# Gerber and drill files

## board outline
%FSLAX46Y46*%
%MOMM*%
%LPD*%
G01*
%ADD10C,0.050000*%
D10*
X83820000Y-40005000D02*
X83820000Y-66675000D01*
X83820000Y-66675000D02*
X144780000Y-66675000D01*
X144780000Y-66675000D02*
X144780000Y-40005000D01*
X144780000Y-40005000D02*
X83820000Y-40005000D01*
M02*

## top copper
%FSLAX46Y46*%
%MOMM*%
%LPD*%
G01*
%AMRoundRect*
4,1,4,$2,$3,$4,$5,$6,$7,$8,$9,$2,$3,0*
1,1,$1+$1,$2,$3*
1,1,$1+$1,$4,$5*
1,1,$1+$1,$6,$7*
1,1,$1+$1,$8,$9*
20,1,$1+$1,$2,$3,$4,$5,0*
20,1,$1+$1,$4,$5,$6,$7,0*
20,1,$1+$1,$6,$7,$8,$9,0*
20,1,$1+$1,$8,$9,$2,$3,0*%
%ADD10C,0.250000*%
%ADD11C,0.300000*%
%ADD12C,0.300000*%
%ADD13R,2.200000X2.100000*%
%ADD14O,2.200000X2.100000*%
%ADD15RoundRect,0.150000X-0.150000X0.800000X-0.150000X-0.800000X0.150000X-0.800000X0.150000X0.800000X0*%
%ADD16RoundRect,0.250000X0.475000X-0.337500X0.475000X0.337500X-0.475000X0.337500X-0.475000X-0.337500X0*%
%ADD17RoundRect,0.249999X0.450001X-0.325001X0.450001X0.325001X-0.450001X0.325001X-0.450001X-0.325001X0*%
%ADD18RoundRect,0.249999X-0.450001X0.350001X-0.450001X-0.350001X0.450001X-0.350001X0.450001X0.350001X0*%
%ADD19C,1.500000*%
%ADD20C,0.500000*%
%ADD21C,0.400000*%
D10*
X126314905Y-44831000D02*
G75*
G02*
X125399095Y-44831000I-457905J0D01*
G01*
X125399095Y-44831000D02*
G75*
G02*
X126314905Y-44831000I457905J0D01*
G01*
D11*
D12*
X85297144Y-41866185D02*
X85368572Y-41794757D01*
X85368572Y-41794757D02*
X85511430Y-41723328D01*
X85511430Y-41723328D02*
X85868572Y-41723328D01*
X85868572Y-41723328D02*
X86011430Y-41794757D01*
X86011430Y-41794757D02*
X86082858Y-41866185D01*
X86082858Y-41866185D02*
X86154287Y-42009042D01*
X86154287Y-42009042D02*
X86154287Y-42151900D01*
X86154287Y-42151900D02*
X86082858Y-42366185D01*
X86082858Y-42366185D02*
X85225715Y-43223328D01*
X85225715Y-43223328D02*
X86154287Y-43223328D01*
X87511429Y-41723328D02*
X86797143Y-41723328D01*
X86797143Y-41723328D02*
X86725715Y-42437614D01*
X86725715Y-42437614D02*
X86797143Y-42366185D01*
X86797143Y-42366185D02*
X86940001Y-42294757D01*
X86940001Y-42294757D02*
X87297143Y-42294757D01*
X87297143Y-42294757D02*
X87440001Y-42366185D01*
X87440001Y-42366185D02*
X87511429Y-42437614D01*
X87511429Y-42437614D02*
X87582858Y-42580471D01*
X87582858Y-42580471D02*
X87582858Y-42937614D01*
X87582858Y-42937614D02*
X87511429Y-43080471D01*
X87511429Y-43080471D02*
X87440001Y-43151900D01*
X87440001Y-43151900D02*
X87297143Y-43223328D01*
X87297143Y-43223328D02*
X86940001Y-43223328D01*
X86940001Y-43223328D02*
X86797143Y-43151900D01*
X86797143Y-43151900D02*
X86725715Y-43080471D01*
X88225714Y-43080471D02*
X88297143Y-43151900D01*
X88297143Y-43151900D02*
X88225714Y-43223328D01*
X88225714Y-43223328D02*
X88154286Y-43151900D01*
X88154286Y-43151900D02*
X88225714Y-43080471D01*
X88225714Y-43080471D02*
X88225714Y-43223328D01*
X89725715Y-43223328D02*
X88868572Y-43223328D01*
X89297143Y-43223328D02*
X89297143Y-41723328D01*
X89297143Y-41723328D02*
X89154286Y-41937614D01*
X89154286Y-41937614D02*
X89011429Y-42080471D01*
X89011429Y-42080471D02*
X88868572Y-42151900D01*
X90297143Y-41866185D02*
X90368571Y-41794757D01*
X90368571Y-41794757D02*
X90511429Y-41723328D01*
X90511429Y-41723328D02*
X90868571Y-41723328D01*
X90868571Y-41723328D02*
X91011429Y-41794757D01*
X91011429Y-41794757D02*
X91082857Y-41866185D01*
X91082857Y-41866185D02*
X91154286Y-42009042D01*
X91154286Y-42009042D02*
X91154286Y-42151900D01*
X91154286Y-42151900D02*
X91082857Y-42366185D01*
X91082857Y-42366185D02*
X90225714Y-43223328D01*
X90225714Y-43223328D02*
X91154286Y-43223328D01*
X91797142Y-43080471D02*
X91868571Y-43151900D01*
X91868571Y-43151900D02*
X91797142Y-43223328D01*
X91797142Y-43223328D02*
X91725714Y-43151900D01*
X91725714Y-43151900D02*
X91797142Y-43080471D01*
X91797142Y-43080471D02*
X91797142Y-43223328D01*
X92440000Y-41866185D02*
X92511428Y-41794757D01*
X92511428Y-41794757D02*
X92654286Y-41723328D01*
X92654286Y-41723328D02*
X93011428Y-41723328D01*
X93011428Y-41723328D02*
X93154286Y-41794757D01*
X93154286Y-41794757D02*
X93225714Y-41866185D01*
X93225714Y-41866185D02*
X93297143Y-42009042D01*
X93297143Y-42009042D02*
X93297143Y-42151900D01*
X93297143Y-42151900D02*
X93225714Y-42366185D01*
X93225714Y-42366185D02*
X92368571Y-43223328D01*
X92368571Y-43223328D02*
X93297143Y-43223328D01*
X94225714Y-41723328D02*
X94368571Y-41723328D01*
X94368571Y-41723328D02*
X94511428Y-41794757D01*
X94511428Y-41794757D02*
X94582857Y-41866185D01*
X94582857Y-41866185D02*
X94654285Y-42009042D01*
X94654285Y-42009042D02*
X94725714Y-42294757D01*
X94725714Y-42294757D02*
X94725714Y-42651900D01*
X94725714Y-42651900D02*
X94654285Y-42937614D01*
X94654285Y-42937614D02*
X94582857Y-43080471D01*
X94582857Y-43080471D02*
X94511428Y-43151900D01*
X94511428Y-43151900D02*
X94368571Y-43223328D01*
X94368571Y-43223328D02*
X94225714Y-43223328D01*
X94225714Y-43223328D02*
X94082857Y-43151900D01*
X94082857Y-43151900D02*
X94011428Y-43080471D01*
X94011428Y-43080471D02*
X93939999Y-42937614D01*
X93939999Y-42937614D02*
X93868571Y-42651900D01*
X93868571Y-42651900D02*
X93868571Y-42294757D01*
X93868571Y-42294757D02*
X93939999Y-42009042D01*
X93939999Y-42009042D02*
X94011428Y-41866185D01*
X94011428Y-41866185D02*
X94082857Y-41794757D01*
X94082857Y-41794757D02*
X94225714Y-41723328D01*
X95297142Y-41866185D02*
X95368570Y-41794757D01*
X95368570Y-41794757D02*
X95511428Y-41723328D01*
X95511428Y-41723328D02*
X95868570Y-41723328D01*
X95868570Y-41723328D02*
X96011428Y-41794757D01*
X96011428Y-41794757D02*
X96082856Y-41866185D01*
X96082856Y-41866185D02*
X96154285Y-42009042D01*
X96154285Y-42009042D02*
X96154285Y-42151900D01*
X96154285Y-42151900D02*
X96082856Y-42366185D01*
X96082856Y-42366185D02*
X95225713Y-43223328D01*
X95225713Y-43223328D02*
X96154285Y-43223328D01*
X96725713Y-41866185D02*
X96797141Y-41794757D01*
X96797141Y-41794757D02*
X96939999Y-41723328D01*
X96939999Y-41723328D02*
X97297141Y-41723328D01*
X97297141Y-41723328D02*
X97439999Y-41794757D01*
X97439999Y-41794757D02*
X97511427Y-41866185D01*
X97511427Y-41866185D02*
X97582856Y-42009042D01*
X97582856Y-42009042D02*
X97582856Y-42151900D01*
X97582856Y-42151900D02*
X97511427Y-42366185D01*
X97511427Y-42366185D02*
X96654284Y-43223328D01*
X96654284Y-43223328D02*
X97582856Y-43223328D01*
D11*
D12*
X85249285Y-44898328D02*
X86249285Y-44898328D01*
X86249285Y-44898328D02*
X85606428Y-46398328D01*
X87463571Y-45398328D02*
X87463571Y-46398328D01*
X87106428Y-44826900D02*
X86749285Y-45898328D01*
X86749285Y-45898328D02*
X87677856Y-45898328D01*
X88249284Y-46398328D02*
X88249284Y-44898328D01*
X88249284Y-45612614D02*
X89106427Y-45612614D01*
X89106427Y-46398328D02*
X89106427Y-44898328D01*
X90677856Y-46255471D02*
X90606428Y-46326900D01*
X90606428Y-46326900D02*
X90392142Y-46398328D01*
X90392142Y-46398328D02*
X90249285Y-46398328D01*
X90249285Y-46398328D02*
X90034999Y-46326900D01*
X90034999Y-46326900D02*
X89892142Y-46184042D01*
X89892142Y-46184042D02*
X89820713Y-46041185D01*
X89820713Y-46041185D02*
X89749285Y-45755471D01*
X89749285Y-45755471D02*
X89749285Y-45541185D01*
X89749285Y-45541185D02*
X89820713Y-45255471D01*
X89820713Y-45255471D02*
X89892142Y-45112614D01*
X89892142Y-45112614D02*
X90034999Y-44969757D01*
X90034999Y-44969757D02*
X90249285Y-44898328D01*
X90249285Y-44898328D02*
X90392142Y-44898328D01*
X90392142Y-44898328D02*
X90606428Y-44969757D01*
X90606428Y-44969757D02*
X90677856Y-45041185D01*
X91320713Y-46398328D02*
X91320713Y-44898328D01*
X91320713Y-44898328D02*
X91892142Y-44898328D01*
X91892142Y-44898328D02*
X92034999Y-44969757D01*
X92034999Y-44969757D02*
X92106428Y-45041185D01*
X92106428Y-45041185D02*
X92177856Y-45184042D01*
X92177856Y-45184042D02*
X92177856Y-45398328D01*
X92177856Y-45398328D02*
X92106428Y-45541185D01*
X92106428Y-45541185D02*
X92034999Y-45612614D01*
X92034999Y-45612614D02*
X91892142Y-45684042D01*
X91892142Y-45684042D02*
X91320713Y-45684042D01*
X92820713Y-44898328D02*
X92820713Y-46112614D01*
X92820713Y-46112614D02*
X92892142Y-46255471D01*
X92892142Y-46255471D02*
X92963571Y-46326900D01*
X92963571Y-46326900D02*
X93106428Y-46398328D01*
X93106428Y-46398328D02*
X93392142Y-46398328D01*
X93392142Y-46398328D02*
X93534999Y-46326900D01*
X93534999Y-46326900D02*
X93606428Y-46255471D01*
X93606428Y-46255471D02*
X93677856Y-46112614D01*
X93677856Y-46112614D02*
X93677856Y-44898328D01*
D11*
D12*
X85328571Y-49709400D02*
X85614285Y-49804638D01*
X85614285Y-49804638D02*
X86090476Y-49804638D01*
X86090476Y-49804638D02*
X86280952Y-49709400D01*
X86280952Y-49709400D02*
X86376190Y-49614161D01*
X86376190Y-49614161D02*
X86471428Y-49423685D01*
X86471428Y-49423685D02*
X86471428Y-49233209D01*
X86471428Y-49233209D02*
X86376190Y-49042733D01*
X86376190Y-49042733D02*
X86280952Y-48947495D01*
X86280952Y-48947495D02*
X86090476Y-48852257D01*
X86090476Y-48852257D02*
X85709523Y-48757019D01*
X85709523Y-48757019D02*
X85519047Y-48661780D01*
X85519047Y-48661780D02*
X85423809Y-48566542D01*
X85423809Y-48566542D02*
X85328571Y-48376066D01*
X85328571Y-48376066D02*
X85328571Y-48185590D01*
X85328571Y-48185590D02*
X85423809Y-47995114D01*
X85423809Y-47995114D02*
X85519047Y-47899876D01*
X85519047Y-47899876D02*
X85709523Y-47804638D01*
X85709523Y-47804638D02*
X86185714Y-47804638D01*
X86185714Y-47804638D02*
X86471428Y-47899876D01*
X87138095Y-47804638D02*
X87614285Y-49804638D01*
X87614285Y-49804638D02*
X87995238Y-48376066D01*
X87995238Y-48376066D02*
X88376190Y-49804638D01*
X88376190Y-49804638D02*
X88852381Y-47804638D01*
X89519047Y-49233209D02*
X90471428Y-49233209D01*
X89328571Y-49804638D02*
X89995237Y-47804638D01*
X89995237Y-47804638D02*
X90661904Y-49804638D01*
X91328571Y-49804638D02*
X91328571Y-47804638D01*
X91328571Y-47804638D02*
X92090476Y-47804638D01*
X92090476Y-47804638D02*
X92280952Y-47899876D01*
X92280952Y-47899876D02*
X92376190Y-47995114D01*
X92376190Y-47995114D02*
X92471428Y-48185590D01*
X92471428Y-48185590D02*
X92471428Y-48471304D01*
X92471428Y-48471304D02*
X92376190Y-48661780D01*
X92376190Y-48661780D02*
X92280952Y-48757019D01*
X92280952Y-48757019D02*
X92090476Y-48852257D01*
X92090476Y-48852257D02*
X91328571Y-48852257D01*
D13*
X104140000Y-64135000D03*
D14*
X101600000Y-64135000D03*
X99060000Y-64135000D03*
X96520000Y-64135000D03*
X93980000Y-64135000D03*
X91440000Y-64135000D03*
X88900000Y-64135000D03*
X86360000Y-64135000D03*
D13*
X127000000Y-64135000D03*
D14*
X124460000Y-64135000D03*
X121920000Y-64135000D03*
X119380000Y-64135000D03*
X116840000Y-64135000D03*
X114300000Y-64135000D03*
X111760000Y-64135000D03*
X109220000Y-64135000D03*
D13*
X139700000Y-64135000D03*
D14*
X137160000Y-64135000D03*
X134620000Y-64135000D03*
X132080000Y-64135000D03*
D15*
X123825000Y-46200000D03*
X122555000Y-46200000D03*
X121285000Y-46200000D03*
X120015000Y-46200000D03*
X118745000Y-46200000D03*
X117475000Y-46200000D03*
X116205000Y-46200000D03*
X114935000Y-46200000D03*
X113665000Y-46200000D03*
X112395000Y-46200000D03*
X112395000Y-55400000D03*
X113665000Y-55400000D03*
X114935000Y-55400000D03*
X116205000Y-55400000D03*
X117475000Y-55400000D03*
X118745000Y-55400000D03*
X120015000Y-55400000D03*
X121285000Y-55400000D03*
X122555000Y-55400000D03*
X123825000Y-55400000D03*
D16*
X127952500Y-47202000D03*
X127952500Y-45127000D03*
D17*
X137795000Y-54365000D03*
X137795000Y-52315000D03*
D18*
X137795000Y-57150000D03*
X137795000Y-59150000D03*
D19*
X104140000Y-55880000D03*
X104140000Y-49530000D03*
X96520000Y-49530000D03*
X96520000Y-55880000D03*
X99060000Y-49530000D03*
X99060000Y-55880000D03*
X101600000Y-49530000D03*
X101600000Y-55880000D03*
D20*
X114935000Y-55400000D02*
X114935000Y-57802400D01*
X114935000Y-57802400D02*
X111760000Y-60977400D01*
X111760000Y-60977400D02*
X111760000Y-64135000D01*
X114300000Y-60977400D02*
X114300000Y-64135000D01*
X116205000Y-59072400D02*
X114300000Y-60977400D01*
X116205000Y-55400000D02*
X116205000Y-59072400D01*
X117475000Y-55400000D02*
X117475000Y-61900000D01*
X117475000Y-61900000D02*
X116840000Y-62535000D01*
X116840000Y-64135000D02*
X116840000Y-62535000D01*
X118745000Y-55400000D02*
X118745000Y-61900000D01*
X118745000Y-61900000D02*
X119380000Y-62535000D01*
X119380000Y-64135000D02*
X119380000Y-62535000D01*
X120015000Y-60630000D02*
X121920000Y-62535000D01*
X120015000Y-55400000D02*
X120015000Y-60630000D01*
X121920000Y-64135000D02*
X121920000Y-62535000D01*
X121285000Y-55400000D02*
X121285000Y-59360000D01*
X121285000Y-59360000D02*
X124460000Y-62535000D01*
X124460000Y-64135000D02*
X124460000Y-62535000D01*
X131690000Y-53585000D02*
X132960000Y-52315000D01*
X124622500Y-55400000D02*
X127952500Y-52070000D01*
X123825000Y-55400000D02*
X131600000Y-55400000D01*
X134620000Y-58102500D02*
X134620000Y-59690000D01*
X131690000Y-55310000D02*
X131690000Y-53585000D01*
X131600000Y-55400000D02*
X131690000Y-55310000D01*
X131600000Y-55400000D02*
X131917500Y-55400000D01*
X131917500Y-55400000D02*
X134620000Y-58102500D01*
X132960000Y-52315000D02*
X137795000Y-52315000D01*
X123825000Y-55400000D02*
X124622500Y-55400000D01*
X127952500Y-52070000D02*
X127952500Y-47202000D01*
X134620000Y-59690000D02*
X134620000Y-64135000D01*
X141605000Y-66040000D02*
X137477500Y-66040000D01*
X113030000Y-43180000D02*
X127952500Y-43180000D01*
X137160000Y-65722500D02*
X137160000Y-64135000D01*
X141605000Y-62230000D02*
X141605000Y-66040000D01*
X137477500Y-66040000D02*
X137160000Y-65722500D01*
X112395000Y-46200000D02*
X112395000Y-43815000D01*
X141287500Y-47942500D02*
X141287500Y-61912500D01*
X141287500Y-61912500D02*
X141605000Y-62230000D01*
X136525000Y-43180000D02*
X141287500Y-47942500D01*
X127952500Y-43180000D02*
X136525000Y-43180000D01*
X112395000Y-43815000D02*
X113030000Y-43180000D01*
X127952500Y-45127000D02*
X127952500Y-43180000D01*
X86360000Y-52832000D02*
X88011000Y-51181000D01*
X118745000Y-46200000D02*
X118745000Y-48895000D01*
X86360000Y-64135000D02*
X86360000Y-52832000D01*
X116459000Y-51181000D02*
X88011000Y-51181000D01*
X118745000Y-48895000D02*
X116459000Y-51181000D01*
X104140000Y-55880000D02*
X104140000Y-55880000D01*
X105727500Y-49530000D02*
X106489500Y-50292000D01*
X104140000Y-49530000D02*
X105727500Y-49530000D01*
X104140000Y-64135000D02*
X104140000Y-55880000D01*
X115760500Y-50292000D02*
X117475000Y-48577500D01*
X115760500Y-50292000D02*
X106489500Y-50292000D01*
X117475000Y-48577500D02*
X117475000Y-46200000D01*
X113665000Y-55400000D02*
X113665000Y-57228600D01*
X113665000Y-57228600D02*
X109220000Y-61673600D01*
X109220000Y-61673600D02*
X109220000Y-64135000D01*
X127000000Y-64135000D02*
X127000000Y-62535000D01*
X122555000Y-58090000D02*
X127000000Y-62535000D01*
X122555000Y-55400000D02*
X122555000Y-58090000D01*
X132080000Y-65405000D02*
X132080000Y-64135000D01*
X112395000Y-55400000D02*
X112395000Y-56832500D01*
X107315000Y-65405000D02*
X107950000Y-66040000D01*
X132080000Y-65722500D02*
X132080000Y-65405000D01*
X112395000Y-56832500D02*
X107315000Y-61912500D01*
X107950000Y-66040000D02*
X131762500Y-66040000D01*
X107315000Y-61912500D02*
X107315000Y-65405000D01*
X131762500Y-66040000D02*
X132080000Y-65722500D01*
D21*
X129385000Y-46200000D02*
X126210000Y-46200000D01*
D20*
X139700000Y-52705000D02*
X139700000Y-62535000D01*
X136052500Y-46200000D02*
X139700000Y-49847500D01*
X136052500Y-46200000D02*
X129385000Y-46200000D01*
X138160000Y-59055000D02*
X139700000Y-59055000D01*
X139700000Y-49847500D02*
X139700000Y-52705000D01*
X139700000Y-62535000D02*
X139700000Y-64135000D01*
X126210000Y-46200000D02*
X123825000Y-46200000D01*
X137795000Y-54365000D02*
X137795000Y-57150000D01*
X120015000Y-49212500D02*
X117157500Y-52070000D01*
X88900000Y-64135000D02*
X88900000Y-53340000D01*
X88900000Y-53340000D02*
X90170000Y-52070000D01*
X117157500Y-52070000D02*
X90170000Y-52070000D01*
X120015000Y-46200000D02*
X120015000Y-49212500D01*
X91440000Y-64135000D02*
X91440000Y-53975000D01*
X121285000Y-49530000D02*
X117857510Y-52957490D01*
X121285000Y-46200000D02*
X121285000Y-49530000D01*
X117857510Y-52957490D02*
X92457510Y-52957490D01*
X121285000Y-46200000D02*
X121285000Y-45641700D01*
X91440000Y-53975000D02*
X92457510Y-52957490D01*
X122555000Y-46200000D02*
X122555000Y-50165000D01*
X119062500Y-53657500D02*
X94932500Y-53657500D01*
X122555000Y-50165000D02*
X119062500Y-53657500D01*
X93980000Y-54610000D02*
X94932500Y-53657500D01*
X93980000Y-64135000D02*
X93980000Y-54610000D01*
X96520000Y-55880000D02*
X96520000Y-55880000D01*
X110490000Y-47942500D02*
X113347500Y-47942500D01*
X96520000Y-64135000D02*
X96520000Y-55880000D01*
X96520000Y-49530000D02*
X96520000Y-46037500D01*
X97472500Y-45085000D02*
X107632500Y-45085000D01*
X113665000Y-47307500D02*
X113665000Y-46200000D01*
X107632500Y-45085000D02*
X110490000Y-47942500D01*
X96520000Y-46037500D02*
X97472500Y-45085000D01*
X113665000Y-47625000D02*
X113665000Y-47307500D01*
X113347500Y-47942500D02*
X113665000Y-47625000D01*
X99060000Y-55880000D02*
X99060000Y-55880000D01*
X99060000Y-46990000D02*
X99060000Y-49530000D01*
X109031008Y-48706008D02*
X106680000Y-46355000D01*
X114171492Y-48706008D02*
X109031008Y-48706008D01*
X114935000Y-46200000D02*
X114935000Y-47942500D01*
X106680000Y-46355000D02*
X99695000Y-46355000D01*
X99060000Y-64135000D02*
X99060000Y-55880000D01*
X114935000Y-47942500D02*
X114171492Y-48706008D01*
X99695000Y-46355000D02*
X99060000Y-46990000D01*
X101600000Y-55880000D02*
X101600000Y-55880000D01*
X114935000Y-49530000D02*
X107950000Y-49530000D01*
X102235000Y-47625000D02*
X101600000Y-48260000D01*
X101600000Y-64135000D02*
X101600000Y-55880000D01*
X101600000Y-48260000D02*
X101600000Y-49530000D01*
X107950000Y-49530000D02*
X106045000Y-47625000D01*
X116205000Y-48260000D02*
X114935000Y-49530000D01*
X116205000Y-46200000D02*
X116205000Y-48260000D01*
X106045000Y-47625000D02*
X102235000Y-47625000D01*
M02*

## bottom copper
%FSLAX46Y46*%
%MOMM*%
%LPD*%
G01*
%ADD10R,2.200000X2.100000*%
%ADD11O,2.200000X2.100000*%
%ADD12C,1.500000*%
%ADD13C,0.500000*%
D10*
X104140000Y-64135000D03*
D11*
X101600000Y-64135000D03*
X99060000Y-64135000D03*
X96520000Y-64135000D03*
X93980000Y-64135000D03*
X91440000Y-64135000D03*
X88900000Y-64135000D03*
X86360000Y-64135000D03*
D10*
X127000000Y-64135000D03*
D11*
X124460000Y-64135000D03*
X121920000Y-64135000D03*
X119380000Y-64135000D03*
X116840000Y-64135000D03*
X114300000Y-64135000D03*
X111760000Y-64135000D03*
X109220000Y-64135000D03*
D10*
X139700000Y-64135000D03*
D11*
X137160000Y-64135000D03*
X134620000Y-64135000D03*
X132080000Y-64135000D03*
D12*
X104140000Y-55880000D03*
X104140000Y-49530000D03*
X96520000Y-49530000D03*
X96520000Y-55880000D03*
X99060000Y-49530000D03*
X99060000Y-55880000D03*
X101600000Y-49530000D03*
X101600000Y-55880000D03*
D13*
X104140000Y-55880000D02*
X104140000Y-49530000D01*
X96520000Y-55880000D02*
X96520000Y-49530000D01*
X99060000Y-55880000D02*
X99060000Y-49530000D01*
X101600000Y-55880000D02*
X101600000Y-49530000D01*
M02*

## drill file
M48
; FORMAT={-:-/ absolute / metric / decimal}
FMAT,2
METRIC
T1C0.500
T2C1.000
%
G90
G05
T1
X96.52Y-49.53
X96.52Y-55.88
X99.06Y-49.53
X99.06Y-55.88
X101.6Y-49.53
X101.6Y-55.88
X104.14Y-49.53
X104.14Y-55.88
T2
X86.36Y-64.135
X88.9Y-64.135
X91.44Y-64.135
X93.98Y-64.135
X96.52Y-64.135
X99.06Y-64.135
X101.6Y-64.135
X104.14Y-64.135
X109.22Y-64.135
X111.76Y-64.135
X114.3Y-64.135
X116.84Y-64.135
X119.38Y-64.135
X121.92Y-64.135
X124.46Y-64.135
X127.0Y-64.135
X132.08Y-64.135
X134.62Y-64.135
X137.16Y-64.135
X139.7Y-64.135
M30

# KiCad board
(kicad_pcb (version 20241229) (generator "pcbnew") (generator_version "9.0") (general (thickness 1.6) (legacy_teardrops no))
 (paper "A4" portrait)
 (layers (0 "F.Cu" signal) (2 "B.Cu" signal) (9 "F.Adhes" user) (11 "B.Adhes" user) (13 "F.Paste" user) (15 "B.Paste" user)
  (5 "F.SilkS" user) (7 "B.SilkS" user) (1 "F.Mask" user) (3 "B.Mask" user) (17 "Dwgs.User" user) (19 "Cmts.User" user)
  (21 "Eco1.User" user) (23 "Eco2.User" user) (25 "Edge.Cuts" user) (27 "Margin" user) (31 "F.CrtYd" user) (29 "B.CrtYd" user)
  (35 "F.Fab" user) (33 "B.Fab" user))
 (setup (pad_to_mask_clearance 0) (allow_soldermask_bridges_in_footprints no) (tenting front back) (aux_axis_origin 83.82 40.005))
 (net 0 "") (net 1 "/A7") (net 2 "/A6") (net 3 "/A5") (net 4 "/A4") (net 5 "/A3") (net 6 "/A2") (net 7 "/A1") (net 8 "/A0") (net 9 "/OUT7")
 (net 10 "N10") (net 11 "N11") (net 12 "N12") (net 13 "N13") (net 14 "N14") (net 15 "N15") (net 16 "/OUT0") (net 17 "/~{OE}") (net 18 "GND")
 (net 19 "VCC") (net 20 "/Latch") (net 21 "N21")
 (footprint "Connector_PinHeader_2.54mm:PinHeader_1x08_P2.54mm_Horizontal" (layer "F.Cu") (at 104.14 64.135 -90)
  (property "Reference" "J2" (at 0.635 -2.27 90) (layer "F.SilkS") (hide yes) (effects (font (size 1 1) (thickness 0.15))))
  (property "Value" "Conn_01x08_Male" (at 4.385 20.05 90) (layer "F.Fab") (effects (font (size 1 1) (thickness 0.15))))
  (pad "1" thru_hole rect (at 0 0 270) (size 2.1 2.2) (drill 1) (layers "*.Cu" "*.Mask") (remove_unused_layers no) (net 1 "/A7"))
  (pad "2" thru_hole oval (at 0 2.54 270) (size 2.1 2.2) (drill 1) (layers "*.Cu" "*.Mask") (remove_unused_layers no) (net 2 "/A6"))
  (pad "3" thru_hole oval (at 0 5.08 270) (size 2.1 2.2) (drill 1) (layers "*.Cu" "*.Mask") (remove_unused_layers no) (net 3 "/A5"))
  (pad "4" thru_hole oval (at 0 7.62 270) (size 2.1 2.2) (drill 1) (layers "*.Cu" "*.Mask") (remove_unused_layers no) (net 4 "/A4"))
  (pad "5" thru_hole oval (at 0 10.16 270) (size 2.1 2.2) (drill 1) (layers "*.Cu" "*.Mask") (remove_unused_layers no) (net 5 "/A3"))
  (pad "6" thru_hole oval (at 0 12.7 270) (size 2.1 2.2) (drill 1) (layers "*.Cu" "*.Mask") (remove_unused_layers no) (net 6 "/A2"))
  (pad "7" thru_hole oval (at 0 15.24 270) (size 2.1 2.2) (drill 1) (layers "*.Cu" "*.Mask") (remove_unused_layers no) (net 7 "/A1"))
  (pad "8" thru_hole oval (at 0 17.78 270) (size 2.1 2.2) (drill 1) (layers "*.Cu" "*.Mask") (remove_unused_layers no) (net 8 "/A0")))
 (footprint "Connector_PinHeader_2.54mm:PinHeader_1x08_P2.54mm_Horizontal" (layer "F.Cu") (at 127 64.135 -90)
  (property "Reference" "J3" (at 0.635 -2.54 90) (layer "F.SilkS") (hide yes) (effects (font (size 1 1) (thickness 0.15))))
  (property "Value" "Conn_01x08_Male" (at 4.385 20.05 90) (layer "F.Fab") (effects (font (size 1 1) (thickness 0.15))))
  (pad "1" thru_hole rect (at 0 0 270) (size 2.1 2.2) (drill 1) (layers "*.Cu" "*.Mask") (remove_unused_layers no) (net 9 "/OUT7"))
  (pad "2" thru_hole oval (at 0 2.54 270) (size 2.1 2.2) (drill 1) (layers "*.Cu" "*.Mask") (remove_unused_layers no) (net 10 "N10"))
  (pad "3" thru_hole oval (at 0 5.08 270) (size 2.1 2.2) (drill 1) (layers "*.Cu" "*.Mask") (remove_unused_layers no) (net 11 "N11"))
  (pad "4" thru_hole oval (at 0 7.62 270) (size 2.1 2.2) (drill 1) (layers "*.Cu" "*.Mask") (remove_unused_layers no) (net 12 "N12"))
  (pad "5" thru_hole oval (at 0 10.16 270) (size 2.1 2.2) (drill 1) (layers "*.Cu" "*.Mask") (remove_unused_layers no) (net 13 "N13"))
  (pad "6" thru_hole oval (at 0 12.7 270) (size 2.1 2.2) (drill 1) (layers "*.Cu" "*.Mask") (remove_unused_layers no) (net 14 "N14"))
  (pad "7" thru_hole oval (at 0 15.24 270) (size 2.1 2.2) (drill 1) (layers "*.Cu" "*.Mask") (remove_unused_layers no) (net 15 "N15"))
  (pad "8" thru_hole oval (at 0 17.78 270) (size 2.1 2.2) (drill 1) (layers "*.Cu" "*.Mask") (remove_unused_layers no) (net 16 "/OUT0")))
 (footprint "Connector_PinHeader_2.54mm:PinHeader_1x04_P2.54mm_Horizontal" (layer "F.Cu") (at 139.7 64.135 -90)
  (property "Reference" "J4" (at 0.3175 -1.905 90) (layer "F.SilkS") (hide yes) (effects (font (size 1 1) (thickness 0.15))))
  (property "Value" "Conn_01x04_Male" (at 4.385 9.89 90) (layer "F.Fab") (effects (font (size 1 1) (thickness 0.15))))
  (pad "1" thru_hole rect (at 0 0 270) (size 2.1 2.2) (drill 1) (layers "*.Cu" "*.Mask") (remove_unused_layers no) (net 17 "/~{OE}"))
  (pad "2" thru_hole oval (at 0 2.54 270) (size 2.1 2.2) (drill 1) (layers "*.Cu" "*.Mask") (remove_unused_layers no) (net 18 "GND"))
  (pad "3" thru_hole oval (at 0 5.08 270) (size 2.1 2.2) (drill 1) (layers "*.Cu" "*.Mask") (remove_unused_layers no) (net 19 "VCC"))
  (pad "4" thru_hole oval (at 0 7.62 270) (size 2.1 2.2) (drill 1) (layers "*.Cu" "*.Mask") (remove_unused_layers no) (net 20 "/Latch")))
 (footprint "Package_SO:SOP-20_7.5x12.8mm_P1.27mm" (layer "F.Cu") (at 118.11 50.8 -90)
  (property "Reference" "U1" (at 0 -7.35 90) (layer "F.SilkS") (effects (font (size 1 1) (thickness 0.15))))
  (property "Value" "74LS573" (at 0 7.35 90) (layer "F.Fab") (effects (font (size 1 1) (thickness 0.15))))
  (pad "1" smd roundrect (at -4.6 -5.715 270) (size 1.9 0.6) (layers "F.Cu" "F.Mask" "F.Paste") (roundrect_rratio 0.25) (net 17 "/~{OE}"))
  (pad "2" smd roundrect (at -4.6 -4.445 270) (size 1.9 0.6) (layers "F.Cu" "F.Mask" "F.Paste") (roundrect_rratio 0.25) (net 5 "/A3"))
  (pad "3" smd roundrect (at -4.6 -3.175 270) (size 1.9 0.6) (layers "F.Cu" "F.Mask" "F.Paste") (roundrect_rratio 0.25) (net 6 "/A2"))
  (pad "4" smd roundrect (at -4.6 -1.905 270) (size 1.9 0.6) (layers "F.Cu" "F.Mask" "F.Paste") (roundrect_rratio 0.25) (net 7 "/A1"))
  (pad "5" smd roundrect (at -4.6 -0.635 270) (size 1.9 0.6) (layers "F.Cu" "F.Mask" "F.Paste") (roundrect_rratio 0.25) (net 8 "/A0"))
  (pad "6" smd roundrect (at -4.6 0.635 270) (size 1.9 0.6) (layers "F.Cu" "F.Mask" "F.Paste") (roundrect_rratio 0.25) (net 1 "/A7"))
  (pad "7" smd roundrect (at -4.6 1.905 270) (size 1.9 0.6) (layers "F.Cu" "F.Mask" "F.Paste") (roundrect_rratio 0.25) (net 2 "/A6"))
  (pad "8" smd roundrect (at -4.6 3.175 270) (size 1.9 0.6) (layers "F.Cu" "F.Mask" "F.Paste") (roundrect_rratio 0.25) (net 3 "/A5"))
  (pad "9" smd roundrect (at -4.6 4.445 270) (size 1.9 0.6) (layers "F.Cu" "F.Mask" "F.Paste") (roundrect_rratio 0.25) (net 4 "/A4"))
  (pad "10" smd roundrect (at -4.6 5.715 270) (size 1.9 0.6) (layers "F.Cu" "F.Mask" "F.Paste") (roundrect_rratio 0.25) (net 18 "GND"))
  (pad "11" smd roundrect (at 4.6 5.715 270) (size 1.9 0.6) (layers "F.Cu" "F.Mask" "F.Paste") (roundrect_rratio 0.25) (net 20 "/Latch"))
  (pad "12" smd roundrect (at 4.6 4.445 270) (size 1.9 0.6) (layers "F.Cu" "F.Mask" "F.Paste") (roundrect_rratio 0.25) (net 16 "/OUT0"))
  (pad "13" smd roundrect (at 4.6 3.175 270) (size 1.9 0.6) (layers "F.Cu" "F.Mask" "F.Paste") (roundrect_rratio 0.25) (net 15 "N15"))
  (pad "14" smd roundrect (at 4.6 1.905 270) (size 1.9 0.6) (layers "F.Cu" "F.Mask" "F.Paste") (roundrect_rratio 0.25) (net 14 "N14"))
  (pad "15" smd roundrect (at 4.6 0.635 270) (size 1.9 0.6) (layers "F.Cu" "F.Mask" "F.Paste") (roundrect_rratio 0.25) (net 13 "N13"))
  (pad "16" smd roundrect (at 4.6 -0.635 270) (size 1.9 0.6) (layers "F.Cu" "F.Mask" "F.Paste") (roundrect_rratio 0.25) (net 12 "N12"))
  (pad "17" smd roundrect (at 4.6 -1.905 270) (size 1.9 0.6) (layers "F.Cu" "F.Mask" "F.Paste") (roundrect_rratio 0.25) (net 11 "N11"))
  (pad "18" smd roundrect (at 4.6 -3.175 270) (size 1.9 0.6) (layers "F.Cu" "F.Mask" "F.Paste") (roundrect_rratio 0.25) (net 10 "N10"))
  (pad "19" smd roundrect (at 4.6 -4.445 270) (size 1.9 0.6) (layers "F.Cu" "F.Mask" "F.Paste") (roundrect_rratio 0.25) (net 9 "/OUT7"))
  (pad "20" smd roundrect (at 4.6 -5.715 270) (size 1.9 0.6) (layers "F.Cu" "F.Mask" "F.Paste") (roundrect_rratio 0.25) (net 19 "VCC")))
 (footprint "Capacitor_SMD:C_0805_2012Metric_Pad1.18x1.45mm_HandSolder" (layer "F.Cu") (at 127.9525 46.1645 90)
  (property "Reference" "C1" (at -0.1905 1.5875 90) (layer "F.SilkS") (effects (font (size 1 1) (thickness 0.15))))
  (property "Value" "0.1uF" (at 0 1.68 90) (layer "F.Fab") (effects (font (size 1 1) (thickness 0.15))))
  (pad "1" smd roundrect (at -1.0375 0 90) (size 1.175 1.45) (layers "F.Cu" "F.Mask" "F.Paste") (roundrect_rratio 0.2127659574)
   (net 19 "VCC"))
  (pad "2" smd roundrect (at 1.0375 0 90) (size 1.175 1.45) (layers "F.Cu" "F.Mask" "F.Paste") (roundrect_rratio 0.2127659574)
   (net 18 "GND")))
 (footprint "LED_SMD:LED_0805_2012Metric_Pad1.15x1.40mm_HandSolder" (layer "F.Cu") (at 137.795 53.34 90)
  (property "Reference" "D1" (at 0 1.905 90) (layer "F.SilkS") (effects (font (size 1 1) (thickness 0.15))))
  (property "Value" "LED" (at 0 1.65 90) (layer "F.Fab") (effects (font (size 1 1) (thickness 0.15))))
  (pad "1" smd roundrect (at -1.025 0 90) (size 1.15 1.4) (layers "F.Cu" "F.Mask" "F.Paste") (roundrect_rratio 0.2173904348) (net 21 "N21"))
  (pad "2" smd roundrect (at 1.025 0 90) (size 1.15 1.4) (layers "F.Cu" "F.Mask" "F.Paste") (roundrect_rratio 0.2173904348) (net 19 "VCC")))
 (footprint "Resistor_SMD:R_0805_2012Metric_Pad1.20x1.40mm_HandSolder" (layer "F.Cu") (at 137.795 58.15 -90)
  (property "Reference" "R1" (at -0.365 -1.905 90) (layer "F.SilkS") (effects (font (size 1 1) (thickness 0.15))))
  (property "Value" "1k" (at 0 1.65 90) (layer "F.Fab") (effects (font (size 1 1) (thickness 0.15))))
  (pad "1" smd roundrect (at -1 0 270) (size 1.2 1.4) (layers "F.Cu" "F.Mask" "F.Paste") (roundrect_rratio 0.2083325) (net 21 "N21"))
  (pad "2" smd roundrect (at 1 0 270) (size 1.2 1.4) (layers "F.Cu" "F.Mask" "F.Paste") (roundrect_rratio 0.2083325) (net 17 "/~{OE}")))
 (gr_circle (center 125.857 44.831) (end 126.314905 44.831) (stroke (width 0.25) (type solid)) (fill no) (layer "F.Cu"))
 (gr_line (start 83.82 40.005) (end 83.82 66.675) (stroke (width 0.05) (type solid)) (layer "Edge.Cuts"))
 (gr_line (start 83.82 66.675) (end 144.78 66.675) (stroke (width 0.05) (type solid)) (layer "Edge.Cuts"))
 (gr_line (start 144.78 66.675) (end 144.78 40.005) (stroke (width 0.05) (type solid)) (layer "Edge.Cuts"))
 (gr_line (start 144.78 40.005) (end 83.82 40.005) (stroke (width 0.05) (type solid)) (layer "Edge.Cuts"))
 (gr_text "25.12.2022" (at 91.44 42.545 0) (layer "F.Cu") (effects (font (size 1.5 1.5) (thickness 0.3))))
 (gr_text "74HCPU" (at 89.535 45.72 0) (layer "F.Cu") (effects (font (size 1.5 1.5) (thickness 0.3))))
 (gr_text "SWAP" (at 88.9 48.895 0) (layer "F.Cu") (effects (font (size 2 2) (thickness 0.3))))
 (segment (start 114.935 55.4) (end 114.935 57.8024) (width 0.5) (layer "F.Cu") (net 15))
 (segment (start 114.935 57.8024) (end 111.76 60.9774) (width 0.5) (layer "F.Cu") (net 15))
 (segment (start 111.76 60.9774) (end 111.76 64.135) (width 0.5) (layer "F.Cu") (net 15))
 (segment (start 114.3 60.9774) (end 114.3 64.135) (width 0.5) (layer "F.Cu") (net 14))
 (segment (start 116.205 59.0724) (end 114.3 60.9774) (width 0.5) (layer "F.Cu") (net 14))
 (segment (start 116.205 55.4) (end 116.205 59.0724) (width 0.5) (layer "F.Cu") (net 14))
 (segment (start 117.475 55.4) (end 117.475 61.9) (width 0.5) (layer "F.Cu") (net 13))
 (segment (start 117.475 61.9) (end 116.84 62.535) (width 0.5) (layer "F.Cu") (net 13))
 (segment (start 116.84 64.135) (end 116.84 62.535) (width 0.5) (layer "F.Cu") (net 13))
 (segment (start 118.745 55.4) (end 118.745 61.9) (width 0.5) (layer "F.Cu") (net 12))
 (segment (start 118.745 61.9) (end 119.38 62.535) (width 0.5) (layer "F.Cu") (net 12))
 (segment (start 119.38 64.135) (end 119.38 62.535) (width 0.5) (layer "F.Cu") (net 12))
 (segment (start 120.015 60.63) (end 121.92 62.535) (width 0.5) (layer "F.Cu") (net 11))
 (segment (start 120.015 55.4) (end 120.015 60.63) (width 0.5) (layer "F.Cu") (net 11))
 (segment (start 121.92 64.135) (end 121.92 62.535) (width 0.5) (layer "F.Cu") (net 11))
 (segment (start 121.285 55.4) (end 121.285 59.36) (width 0.5) (layer "F.Cu") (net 10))
 (segment (start 121.285 59.36) (end 124.46 62.535) (width 0.5) (layer "F.Cu") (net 10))
 (segment (start 124.46 64.135) (end 124.46 62.535) (width 0.5) (layer "F.Cu") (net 10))
 (segment (start 131.69 53.585) (end 132.96 52.315) (width 0.5) (layer "F.Cu") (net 19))
 (segment (start 124.6225 55.4) (end 127.9525 52.07) (width 0.5) (layer "F.Cu") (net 19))
 (segment (start 123.825 55.4) (end 131.6 55.4) (width 0.5) (layer "F.Cu") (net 19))
 (segment (start 134.62 58.1025) (end 134.62 59.69) (width 0.5) (layer "F.Cu") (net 19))
 (segment (start 131.69 55.31) (end 131.69 53.585) (width 0.5) (layer "F.Cu") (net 19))
 (segment (start 131.6 55.4) (end 131.69 55.31) (width 0.5) (layer "F.Cu") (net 19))
 (segment (start 131.6 55.4) (end 131.9175 55.4) (width 0.5) (layer "F.Cu") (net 19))
 (segment (start 131.9175 55.4) (end 134.62 58.1025) (width 0.5) (layer "F.Cu") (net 19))
 (segment (start 132.96 52.315) (end 137.795 52.315) (width 0.5) (layer "F.Cu") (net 19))
 (segment (start 123.825 55.4) (end 124.6225 55.4) (width 0.5) (layer "F.Cu") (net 19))
 (segment (start 127.9525 52.07) (end 127.9525 47.202) (width 0.5) (layer "F.Cu") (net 19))
 (segment (start 134.62 59.69) (end 134.62 64.135) (width 0.5) (layer "F.Cu") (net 19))
 (segment (start 141.605 66.04) (end 137.4775 66.04) (width 0.5) (layer "F.Cu") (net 18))
 (segment (start 113.03 43.18) (end 127.9525 43.18) (width 0.5) (layer "F.Cu") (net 18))
 (segment (start 137.16 65.7225) (end 137.16 64.135) (width 0.5) (layer "F.Cu") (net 18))
 (segment (start 141.605 62.23) (end 141.605 66.04) (width 0.5) (layer "F.Cu") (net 18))
 (segment (start 137.4775 66.04) (end 137.16 65.7225) (width 0.5) (layer "F.Cu") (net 18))
 (segment (start 112.395 46.2) (end 112.395 43.815) (width 0.5) (layer "F.Cu") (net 18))
 (segment (start 141.2875 47.9425) (end 141.2875 61.9125) (width 0.5) (layer "F.Cu") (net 18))
 (segment (start 141.2875 61.9125) (end 141.605 62.23) (width 0.5) (layer "F.Cu") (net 18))
 (segment (start 136.525 43.18) (end 141.2875 47.9425) (width 0.5) (layer "F.Cu") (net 18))
 (segment (start 127.9525 43.18) (end 136.525 43.18) (width 0.5) (layer "F.Cu") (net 18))
 (segment (start 112.395 43.815) (end 113.03 43.18) (width 0.5) (layer "F.Cu") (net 18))
 (segment (start 127.9525 45.127) (end 127.9525 43.18) (width 0.5) (layer "F.Cu") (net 18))
 (segment (start 86.36 52.832) (end 88.011 51.181) (width 0.5) (layer "F.Cu") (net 8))
 (segment (start 118.745 46.2) (end 118.745 48.895) (width 0.5) (layer "F.Cu") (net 8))
 (segment (start 86.36 64.135) (end 86.36 52.832) (width 0.5) (layer "F.Cu") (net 8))
 (segment (start 116.459 51.181) (end 88.011 51.181) (width 0.5) (layer "F.Cu") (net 8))
 (segment (start 118.745 48.895) (end 116.459 51.181) (width 0.5) (layer "F.Cu") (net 8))
 (segment (start 104.14 55.88) (end 104.14 55.88) (width 0.5) (layer "F.Cu") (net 1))
 (segment (start 105.7275 49.53) (end 106.4895 50.292) (width 0.5) (layer "F.Cu") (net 1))
 (segment (start 104.14 49.53) (end 105.7275 49.53) (width 0.5) (layer "F.Cu") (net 1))
 (segment (start 104.14 64.135) (end 104.14 55.88) (width 0.5) (layer "F.Cu") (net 1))
 (segment (start 115.7605 50.292) (end 117.475 48.5775) (width 0.5) (layer "F.Cu") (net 1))
 (segment (start 115.7605 50.292) (end 106.4895 50.292) (width 0.5) (layer "F.Cu") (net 1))
 (segment (start 117.475 48.5775) (end 117.475 46.2) (width 0.5) (layer "F.Cu") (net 1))
 (via (at 104.14 55.88) (size 1.5) (drill 0.5) (layers "F.Cu" "B.Cu") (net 1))
 (via (at 104.14 49.53) (size 1.5) (drill 0.5) (layers "F.Cu" "B.Cu") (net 1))
 (segment (start 104.14 55.88) (end 104.14 49.53) (width 0.5) (layer "B.Cu") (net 1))
 (segment (start 113.665 55.4) (end 113.665 57.2286) (width 0.5) (layer "F.Cu") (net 16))
 (segment (start 113.665 57.2286) (end 109.22 61.6736) (width 0.5) (layer "F.Cu") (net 16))
 (segment (start 109.22 61.6736) (end 109.22 64.135) (width 0.5) (layer "F.Cu") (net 16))
 (segment (start 127 64.135) (end 127 62.535) (width 0.5) (layer "F.Cu") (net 9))
 (segment (start 122.555 58.09) (end 127 62.535) (width 0.5) (layer "F.Cu") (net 9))
 (segment (start 122.555 55.4) (end 122.555 58.09) (width 0.5) (layer "F.Cu") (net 9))
 (segment (start 132.08 65.405) (end 132.08 64.135) (width 0.5) (layer "F.Cu") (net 20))
 (segment (start 112.395 55.4) (end 112.395 56.8325) (width 0.5) (layer "F.Cu") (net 20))
 (segment (start 107.315 65.405) (end 107.95 66.04) (width 0.5) (layer "F.Cu") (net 20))
 (segment (start 132.08 65.7225) (end 132.08 65.405) (width 0.5) (layer "F.Cu") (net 20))
 (segment (start 112.395 56.8325) (end 107.315 61.9125) (width 0.5) (layer "F.Cu") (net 20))
 (segment (start 107.95 66.04) (end 131.7625 66.04) (width 0.5) (layer "F.Cu") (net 20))
 (segment (start 107.315 61.9125) (end 107.315 65.405) (width 0.5) (layer "F.Cu") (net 20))
 (segment (start 131.7625 66.04) (end 132.08 65.7225) (width 0.5) (layer "F.Cu") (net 20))
 (segment (start 129.385 46.2) (end 126.21 46.2) (width 0.4) (layer "F.Cu") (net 17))
 (segment (start 139.7 52.705) (end 139.7 62.535) (width 0.5) (layer "F.Cu") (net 17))
 (segment (start 136.0525 46.2) (end 139.7 49.8475) (width 0.5) (layer "F.Cu") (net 17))
 (segment (start 136.0525 46.2) (end 129.385 46.2) (width 0.5) (layer "F.Cu") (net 17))
 (segment (start 138.16 59.055) (end 139.7 59.055) (width 0.5) (layer "F.Cu") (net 17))
 (segment (start 139.7 49.8475) (end 139.7 52.705) (width 0.5) (layer "F.Cu") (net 17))
 (segment (start 139.7 62.535) (end 139.7 64.135) (width 0.5) (layer "F.Cu") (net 17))
 (segment (start 126.21 46.2) (end 123.825 46.2) (width 0.5) (layer "F.Cu") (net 17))
 (segment (start 137.795 54.365) (end 137.795 57.15) (width 0.5) (layer "F.Cu") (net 21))
 (segment (start 120.015 49.2125) (end 117.1575 52.07) (width 0.5) (layer "F.Cu") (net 7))
 (segment (start 88.9 64.135) (end 88.9 53.34) (width 0.5) (layer "F.Cu") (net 7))
 (segment (start 88.9 53.34) (end 90.17 52.07) (width 0.5) (layer "F.Cu") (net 7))
 (segment (start 117.1575 52.07) (end 90.17 52.07) (width 0.5) (layer "F.Cu") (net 7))
 (segment (start 120.015 46.2) (end 120.015 49.2125) (width 0.5) (layer "F.Cu") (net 7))
 (segment (start 91.44 64.135) (end 91.44 53.975) (width 0.5) (layer "F.Cu") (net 6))
 (segment (start 121.285 49.53) (end 117.85751 52.95749) (width 0.5) (layer "F.Cu") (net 6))
 (segment (start 121.285 46.2) (end 121.285 49.53) (width 0.5) (layer "F.Cu") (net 6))
 (segment (start 117.85751 52.95749) (end 92.45751 52.95749) (width 0.5) (layer "F.Cu") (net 6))
 (segment (start 121.285 46.2) (end 121.285 45.6417) (width 0.5) (layer "F.Cu") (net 6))
 (segment (start 91.44 53.975) (end 92.45751 52.95749) (width 0.5) (layer "F.Cu") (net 6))
 (segment (start 122.555 46.2) (end 122.555 50.165) (width 0.5) (layer "F.Cu") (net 5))
 (segment (start 119.0625 53.6575) (end 94.9325 53.6575) (width 0.5) (layer "F.Cu") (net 5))
 (segment (start 122.555 50.165) (end 119.0625 53.6575) (width 0.5) (layer "F.Cu") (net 5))
 (segment (start 93.98 54.61) (end 94.9325 53.6575) (width 0.5) (layer "F.Cu") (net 5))
 (segment (start 93.98 64.135) (end 93.98 54.61) (width 0.5) (layer "F.Cu") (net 5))
 (segment (start 96.52 55.88) (end 96.52 55.88) (width 0.5) (layer "F.Cu") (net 4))
 (segment (start 110.49 47.9425) (end 113.3475 47.9425) (width 0.5) (layer "F.Cu") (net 4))
 (segment (start 96.52 64.135) (end 96.52 55.88) (width 0.5) (layer "F.Cu") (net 4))
 (segment (start 96.52 49.53) (end 96.52 46.0375) (width 0.5) (layer "F.Cu") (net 4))
 (segment (start 97.4725 45.085) (end 107.6325 45.085) (width 0.5) (layer "F.Cu") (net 4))
 (segment (start 113.665 47.3075) (end 113.665 46.2) (width 0.5) (layer "F.Cu") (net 4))
 (segment (start 107.6325 45.085) (end 110.49 47.9425) (width 0.5) (layer "F.Cu") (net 4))
 (segment (start 96.52 46.0375) (end 97.4725 45.085) (width 0.5) (layer "F.Cu") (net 4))
 (segment (start 113.665 47.625) (end 113.665 47.3075) (width 0.5) (layer "F.Cu") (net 4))
 (segment (start 113.3475 47.9425) (end 113.665 47.625) (width 0.5) (layer "F.Cu") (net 4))
 (via (at 96.52 49.53) (size 1.5) (drill 0.5) (layers "F.Cu" "B.Cu") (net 4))
 (via (at 96.52 55.88) (size 1.5) (drill 0.5) (layers "F.Cu" "B.Cu") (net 4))
 (segment (start 96.52 55.88) (end 96.52 49.53) (width 0.5) (layer "B.Cu") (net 4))
 (segment (start 99.06 55.88) (end 99.06 55.88) (width 0.5) (layer "F.Cu") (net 3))
 (segment (start 99.06 46.99) (end 99.06 49.53) (width 0.5) (layer "F.Cu") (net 3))
 (segment (start 109.031008 48.706008) (end 106.68 46.355) (width 0.5) (layer "F.Cu") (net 3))
 (segment (start 114.171492 48.706008) (end 109.031008 48.706008) (width 0.5) (layer "F.Cu") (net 3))
 (segment (start 114.935 46.2) (end 114.935 47.9425) (width 0.5) (layer "F.Cu") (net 3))
 (segment (start 106.68 46.355) (end 99.695 46.355) (width 0.5) (layer "F.Cu") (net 3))
 (segment (start 99.06 64.135) (end 99.06 55.88) (width 0.5) (layer "F.Cu") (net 3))
 (segment (start 114.935 47.9425) (end 114.171492 48.706008) (width 0.5) (layer "F.Cu") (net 3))
 (segment (start 99.695 46.355) (end 99.06 46.99) (width 0.5) (layer "F.Cu") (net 3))
 (via (at 99.06 49.53) (size 1.5) (drill 0.5) (layers "F.Cu" "B.Cu") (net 3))
 (via (at 99.06 55.88) (size 1.5) (drill 0.5) (layers "F.Cu" "B.Cu") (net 3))
 (segment (start 99.06 55.88) (end 99.06 49.53) (width 0.5) (layer "B.Cu") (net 3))
 (segment (start 101.6 55.88) (end 101.6 55.88) (width 0.5) (layer "F.Cu") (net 2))
 (segment (start 114.935 49.53) (end 107.95 49.53) (width 0.5) (layer "F.Cu") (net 2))
 (segment (start 102.235 47.625) (end 101.6 48.26) (width 0.5) (layer "F.Cu") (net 2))
 (segment (start 101.6 64.135) (end 101.6 55.88) (width 0.5) (layer "F.Cu") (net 2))
 (segment (start 101.6 48.26) (end 101.6 49.53) (width 0.5) (layer "F.Cu") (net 2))
 (segment (start 107.95 49.53) (end 106.045 47.625) (width 0.5) (layer "F.Cu") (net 2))
 (segment (start 116.205 48.26) (end 114.935 49.53) (width 0.5) (layer "F.Cu") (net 2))
 (segment (start 116.205 46.2) (end 116.205 48.26) (width 0.5) (layer "F.Cu") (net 2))
 (segment (start 106.045 47.625) (end 102.235 47.625) (width 0.5) (layer "F.Cu") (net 2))
 (via (at 101.6 49.53) (size 1.5) (drill 0.5) (layers "F.Cu" "B.Cu") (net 2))
 (via (at 101.6 55.88) (size 1.5) (drill 0.5) (layers "F.Cu" "B.Cu") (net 2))
 (segment (start 101.6 55.88) (end 101.6 49.53) (width 0.5) (layer "B.Cu") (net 2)))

